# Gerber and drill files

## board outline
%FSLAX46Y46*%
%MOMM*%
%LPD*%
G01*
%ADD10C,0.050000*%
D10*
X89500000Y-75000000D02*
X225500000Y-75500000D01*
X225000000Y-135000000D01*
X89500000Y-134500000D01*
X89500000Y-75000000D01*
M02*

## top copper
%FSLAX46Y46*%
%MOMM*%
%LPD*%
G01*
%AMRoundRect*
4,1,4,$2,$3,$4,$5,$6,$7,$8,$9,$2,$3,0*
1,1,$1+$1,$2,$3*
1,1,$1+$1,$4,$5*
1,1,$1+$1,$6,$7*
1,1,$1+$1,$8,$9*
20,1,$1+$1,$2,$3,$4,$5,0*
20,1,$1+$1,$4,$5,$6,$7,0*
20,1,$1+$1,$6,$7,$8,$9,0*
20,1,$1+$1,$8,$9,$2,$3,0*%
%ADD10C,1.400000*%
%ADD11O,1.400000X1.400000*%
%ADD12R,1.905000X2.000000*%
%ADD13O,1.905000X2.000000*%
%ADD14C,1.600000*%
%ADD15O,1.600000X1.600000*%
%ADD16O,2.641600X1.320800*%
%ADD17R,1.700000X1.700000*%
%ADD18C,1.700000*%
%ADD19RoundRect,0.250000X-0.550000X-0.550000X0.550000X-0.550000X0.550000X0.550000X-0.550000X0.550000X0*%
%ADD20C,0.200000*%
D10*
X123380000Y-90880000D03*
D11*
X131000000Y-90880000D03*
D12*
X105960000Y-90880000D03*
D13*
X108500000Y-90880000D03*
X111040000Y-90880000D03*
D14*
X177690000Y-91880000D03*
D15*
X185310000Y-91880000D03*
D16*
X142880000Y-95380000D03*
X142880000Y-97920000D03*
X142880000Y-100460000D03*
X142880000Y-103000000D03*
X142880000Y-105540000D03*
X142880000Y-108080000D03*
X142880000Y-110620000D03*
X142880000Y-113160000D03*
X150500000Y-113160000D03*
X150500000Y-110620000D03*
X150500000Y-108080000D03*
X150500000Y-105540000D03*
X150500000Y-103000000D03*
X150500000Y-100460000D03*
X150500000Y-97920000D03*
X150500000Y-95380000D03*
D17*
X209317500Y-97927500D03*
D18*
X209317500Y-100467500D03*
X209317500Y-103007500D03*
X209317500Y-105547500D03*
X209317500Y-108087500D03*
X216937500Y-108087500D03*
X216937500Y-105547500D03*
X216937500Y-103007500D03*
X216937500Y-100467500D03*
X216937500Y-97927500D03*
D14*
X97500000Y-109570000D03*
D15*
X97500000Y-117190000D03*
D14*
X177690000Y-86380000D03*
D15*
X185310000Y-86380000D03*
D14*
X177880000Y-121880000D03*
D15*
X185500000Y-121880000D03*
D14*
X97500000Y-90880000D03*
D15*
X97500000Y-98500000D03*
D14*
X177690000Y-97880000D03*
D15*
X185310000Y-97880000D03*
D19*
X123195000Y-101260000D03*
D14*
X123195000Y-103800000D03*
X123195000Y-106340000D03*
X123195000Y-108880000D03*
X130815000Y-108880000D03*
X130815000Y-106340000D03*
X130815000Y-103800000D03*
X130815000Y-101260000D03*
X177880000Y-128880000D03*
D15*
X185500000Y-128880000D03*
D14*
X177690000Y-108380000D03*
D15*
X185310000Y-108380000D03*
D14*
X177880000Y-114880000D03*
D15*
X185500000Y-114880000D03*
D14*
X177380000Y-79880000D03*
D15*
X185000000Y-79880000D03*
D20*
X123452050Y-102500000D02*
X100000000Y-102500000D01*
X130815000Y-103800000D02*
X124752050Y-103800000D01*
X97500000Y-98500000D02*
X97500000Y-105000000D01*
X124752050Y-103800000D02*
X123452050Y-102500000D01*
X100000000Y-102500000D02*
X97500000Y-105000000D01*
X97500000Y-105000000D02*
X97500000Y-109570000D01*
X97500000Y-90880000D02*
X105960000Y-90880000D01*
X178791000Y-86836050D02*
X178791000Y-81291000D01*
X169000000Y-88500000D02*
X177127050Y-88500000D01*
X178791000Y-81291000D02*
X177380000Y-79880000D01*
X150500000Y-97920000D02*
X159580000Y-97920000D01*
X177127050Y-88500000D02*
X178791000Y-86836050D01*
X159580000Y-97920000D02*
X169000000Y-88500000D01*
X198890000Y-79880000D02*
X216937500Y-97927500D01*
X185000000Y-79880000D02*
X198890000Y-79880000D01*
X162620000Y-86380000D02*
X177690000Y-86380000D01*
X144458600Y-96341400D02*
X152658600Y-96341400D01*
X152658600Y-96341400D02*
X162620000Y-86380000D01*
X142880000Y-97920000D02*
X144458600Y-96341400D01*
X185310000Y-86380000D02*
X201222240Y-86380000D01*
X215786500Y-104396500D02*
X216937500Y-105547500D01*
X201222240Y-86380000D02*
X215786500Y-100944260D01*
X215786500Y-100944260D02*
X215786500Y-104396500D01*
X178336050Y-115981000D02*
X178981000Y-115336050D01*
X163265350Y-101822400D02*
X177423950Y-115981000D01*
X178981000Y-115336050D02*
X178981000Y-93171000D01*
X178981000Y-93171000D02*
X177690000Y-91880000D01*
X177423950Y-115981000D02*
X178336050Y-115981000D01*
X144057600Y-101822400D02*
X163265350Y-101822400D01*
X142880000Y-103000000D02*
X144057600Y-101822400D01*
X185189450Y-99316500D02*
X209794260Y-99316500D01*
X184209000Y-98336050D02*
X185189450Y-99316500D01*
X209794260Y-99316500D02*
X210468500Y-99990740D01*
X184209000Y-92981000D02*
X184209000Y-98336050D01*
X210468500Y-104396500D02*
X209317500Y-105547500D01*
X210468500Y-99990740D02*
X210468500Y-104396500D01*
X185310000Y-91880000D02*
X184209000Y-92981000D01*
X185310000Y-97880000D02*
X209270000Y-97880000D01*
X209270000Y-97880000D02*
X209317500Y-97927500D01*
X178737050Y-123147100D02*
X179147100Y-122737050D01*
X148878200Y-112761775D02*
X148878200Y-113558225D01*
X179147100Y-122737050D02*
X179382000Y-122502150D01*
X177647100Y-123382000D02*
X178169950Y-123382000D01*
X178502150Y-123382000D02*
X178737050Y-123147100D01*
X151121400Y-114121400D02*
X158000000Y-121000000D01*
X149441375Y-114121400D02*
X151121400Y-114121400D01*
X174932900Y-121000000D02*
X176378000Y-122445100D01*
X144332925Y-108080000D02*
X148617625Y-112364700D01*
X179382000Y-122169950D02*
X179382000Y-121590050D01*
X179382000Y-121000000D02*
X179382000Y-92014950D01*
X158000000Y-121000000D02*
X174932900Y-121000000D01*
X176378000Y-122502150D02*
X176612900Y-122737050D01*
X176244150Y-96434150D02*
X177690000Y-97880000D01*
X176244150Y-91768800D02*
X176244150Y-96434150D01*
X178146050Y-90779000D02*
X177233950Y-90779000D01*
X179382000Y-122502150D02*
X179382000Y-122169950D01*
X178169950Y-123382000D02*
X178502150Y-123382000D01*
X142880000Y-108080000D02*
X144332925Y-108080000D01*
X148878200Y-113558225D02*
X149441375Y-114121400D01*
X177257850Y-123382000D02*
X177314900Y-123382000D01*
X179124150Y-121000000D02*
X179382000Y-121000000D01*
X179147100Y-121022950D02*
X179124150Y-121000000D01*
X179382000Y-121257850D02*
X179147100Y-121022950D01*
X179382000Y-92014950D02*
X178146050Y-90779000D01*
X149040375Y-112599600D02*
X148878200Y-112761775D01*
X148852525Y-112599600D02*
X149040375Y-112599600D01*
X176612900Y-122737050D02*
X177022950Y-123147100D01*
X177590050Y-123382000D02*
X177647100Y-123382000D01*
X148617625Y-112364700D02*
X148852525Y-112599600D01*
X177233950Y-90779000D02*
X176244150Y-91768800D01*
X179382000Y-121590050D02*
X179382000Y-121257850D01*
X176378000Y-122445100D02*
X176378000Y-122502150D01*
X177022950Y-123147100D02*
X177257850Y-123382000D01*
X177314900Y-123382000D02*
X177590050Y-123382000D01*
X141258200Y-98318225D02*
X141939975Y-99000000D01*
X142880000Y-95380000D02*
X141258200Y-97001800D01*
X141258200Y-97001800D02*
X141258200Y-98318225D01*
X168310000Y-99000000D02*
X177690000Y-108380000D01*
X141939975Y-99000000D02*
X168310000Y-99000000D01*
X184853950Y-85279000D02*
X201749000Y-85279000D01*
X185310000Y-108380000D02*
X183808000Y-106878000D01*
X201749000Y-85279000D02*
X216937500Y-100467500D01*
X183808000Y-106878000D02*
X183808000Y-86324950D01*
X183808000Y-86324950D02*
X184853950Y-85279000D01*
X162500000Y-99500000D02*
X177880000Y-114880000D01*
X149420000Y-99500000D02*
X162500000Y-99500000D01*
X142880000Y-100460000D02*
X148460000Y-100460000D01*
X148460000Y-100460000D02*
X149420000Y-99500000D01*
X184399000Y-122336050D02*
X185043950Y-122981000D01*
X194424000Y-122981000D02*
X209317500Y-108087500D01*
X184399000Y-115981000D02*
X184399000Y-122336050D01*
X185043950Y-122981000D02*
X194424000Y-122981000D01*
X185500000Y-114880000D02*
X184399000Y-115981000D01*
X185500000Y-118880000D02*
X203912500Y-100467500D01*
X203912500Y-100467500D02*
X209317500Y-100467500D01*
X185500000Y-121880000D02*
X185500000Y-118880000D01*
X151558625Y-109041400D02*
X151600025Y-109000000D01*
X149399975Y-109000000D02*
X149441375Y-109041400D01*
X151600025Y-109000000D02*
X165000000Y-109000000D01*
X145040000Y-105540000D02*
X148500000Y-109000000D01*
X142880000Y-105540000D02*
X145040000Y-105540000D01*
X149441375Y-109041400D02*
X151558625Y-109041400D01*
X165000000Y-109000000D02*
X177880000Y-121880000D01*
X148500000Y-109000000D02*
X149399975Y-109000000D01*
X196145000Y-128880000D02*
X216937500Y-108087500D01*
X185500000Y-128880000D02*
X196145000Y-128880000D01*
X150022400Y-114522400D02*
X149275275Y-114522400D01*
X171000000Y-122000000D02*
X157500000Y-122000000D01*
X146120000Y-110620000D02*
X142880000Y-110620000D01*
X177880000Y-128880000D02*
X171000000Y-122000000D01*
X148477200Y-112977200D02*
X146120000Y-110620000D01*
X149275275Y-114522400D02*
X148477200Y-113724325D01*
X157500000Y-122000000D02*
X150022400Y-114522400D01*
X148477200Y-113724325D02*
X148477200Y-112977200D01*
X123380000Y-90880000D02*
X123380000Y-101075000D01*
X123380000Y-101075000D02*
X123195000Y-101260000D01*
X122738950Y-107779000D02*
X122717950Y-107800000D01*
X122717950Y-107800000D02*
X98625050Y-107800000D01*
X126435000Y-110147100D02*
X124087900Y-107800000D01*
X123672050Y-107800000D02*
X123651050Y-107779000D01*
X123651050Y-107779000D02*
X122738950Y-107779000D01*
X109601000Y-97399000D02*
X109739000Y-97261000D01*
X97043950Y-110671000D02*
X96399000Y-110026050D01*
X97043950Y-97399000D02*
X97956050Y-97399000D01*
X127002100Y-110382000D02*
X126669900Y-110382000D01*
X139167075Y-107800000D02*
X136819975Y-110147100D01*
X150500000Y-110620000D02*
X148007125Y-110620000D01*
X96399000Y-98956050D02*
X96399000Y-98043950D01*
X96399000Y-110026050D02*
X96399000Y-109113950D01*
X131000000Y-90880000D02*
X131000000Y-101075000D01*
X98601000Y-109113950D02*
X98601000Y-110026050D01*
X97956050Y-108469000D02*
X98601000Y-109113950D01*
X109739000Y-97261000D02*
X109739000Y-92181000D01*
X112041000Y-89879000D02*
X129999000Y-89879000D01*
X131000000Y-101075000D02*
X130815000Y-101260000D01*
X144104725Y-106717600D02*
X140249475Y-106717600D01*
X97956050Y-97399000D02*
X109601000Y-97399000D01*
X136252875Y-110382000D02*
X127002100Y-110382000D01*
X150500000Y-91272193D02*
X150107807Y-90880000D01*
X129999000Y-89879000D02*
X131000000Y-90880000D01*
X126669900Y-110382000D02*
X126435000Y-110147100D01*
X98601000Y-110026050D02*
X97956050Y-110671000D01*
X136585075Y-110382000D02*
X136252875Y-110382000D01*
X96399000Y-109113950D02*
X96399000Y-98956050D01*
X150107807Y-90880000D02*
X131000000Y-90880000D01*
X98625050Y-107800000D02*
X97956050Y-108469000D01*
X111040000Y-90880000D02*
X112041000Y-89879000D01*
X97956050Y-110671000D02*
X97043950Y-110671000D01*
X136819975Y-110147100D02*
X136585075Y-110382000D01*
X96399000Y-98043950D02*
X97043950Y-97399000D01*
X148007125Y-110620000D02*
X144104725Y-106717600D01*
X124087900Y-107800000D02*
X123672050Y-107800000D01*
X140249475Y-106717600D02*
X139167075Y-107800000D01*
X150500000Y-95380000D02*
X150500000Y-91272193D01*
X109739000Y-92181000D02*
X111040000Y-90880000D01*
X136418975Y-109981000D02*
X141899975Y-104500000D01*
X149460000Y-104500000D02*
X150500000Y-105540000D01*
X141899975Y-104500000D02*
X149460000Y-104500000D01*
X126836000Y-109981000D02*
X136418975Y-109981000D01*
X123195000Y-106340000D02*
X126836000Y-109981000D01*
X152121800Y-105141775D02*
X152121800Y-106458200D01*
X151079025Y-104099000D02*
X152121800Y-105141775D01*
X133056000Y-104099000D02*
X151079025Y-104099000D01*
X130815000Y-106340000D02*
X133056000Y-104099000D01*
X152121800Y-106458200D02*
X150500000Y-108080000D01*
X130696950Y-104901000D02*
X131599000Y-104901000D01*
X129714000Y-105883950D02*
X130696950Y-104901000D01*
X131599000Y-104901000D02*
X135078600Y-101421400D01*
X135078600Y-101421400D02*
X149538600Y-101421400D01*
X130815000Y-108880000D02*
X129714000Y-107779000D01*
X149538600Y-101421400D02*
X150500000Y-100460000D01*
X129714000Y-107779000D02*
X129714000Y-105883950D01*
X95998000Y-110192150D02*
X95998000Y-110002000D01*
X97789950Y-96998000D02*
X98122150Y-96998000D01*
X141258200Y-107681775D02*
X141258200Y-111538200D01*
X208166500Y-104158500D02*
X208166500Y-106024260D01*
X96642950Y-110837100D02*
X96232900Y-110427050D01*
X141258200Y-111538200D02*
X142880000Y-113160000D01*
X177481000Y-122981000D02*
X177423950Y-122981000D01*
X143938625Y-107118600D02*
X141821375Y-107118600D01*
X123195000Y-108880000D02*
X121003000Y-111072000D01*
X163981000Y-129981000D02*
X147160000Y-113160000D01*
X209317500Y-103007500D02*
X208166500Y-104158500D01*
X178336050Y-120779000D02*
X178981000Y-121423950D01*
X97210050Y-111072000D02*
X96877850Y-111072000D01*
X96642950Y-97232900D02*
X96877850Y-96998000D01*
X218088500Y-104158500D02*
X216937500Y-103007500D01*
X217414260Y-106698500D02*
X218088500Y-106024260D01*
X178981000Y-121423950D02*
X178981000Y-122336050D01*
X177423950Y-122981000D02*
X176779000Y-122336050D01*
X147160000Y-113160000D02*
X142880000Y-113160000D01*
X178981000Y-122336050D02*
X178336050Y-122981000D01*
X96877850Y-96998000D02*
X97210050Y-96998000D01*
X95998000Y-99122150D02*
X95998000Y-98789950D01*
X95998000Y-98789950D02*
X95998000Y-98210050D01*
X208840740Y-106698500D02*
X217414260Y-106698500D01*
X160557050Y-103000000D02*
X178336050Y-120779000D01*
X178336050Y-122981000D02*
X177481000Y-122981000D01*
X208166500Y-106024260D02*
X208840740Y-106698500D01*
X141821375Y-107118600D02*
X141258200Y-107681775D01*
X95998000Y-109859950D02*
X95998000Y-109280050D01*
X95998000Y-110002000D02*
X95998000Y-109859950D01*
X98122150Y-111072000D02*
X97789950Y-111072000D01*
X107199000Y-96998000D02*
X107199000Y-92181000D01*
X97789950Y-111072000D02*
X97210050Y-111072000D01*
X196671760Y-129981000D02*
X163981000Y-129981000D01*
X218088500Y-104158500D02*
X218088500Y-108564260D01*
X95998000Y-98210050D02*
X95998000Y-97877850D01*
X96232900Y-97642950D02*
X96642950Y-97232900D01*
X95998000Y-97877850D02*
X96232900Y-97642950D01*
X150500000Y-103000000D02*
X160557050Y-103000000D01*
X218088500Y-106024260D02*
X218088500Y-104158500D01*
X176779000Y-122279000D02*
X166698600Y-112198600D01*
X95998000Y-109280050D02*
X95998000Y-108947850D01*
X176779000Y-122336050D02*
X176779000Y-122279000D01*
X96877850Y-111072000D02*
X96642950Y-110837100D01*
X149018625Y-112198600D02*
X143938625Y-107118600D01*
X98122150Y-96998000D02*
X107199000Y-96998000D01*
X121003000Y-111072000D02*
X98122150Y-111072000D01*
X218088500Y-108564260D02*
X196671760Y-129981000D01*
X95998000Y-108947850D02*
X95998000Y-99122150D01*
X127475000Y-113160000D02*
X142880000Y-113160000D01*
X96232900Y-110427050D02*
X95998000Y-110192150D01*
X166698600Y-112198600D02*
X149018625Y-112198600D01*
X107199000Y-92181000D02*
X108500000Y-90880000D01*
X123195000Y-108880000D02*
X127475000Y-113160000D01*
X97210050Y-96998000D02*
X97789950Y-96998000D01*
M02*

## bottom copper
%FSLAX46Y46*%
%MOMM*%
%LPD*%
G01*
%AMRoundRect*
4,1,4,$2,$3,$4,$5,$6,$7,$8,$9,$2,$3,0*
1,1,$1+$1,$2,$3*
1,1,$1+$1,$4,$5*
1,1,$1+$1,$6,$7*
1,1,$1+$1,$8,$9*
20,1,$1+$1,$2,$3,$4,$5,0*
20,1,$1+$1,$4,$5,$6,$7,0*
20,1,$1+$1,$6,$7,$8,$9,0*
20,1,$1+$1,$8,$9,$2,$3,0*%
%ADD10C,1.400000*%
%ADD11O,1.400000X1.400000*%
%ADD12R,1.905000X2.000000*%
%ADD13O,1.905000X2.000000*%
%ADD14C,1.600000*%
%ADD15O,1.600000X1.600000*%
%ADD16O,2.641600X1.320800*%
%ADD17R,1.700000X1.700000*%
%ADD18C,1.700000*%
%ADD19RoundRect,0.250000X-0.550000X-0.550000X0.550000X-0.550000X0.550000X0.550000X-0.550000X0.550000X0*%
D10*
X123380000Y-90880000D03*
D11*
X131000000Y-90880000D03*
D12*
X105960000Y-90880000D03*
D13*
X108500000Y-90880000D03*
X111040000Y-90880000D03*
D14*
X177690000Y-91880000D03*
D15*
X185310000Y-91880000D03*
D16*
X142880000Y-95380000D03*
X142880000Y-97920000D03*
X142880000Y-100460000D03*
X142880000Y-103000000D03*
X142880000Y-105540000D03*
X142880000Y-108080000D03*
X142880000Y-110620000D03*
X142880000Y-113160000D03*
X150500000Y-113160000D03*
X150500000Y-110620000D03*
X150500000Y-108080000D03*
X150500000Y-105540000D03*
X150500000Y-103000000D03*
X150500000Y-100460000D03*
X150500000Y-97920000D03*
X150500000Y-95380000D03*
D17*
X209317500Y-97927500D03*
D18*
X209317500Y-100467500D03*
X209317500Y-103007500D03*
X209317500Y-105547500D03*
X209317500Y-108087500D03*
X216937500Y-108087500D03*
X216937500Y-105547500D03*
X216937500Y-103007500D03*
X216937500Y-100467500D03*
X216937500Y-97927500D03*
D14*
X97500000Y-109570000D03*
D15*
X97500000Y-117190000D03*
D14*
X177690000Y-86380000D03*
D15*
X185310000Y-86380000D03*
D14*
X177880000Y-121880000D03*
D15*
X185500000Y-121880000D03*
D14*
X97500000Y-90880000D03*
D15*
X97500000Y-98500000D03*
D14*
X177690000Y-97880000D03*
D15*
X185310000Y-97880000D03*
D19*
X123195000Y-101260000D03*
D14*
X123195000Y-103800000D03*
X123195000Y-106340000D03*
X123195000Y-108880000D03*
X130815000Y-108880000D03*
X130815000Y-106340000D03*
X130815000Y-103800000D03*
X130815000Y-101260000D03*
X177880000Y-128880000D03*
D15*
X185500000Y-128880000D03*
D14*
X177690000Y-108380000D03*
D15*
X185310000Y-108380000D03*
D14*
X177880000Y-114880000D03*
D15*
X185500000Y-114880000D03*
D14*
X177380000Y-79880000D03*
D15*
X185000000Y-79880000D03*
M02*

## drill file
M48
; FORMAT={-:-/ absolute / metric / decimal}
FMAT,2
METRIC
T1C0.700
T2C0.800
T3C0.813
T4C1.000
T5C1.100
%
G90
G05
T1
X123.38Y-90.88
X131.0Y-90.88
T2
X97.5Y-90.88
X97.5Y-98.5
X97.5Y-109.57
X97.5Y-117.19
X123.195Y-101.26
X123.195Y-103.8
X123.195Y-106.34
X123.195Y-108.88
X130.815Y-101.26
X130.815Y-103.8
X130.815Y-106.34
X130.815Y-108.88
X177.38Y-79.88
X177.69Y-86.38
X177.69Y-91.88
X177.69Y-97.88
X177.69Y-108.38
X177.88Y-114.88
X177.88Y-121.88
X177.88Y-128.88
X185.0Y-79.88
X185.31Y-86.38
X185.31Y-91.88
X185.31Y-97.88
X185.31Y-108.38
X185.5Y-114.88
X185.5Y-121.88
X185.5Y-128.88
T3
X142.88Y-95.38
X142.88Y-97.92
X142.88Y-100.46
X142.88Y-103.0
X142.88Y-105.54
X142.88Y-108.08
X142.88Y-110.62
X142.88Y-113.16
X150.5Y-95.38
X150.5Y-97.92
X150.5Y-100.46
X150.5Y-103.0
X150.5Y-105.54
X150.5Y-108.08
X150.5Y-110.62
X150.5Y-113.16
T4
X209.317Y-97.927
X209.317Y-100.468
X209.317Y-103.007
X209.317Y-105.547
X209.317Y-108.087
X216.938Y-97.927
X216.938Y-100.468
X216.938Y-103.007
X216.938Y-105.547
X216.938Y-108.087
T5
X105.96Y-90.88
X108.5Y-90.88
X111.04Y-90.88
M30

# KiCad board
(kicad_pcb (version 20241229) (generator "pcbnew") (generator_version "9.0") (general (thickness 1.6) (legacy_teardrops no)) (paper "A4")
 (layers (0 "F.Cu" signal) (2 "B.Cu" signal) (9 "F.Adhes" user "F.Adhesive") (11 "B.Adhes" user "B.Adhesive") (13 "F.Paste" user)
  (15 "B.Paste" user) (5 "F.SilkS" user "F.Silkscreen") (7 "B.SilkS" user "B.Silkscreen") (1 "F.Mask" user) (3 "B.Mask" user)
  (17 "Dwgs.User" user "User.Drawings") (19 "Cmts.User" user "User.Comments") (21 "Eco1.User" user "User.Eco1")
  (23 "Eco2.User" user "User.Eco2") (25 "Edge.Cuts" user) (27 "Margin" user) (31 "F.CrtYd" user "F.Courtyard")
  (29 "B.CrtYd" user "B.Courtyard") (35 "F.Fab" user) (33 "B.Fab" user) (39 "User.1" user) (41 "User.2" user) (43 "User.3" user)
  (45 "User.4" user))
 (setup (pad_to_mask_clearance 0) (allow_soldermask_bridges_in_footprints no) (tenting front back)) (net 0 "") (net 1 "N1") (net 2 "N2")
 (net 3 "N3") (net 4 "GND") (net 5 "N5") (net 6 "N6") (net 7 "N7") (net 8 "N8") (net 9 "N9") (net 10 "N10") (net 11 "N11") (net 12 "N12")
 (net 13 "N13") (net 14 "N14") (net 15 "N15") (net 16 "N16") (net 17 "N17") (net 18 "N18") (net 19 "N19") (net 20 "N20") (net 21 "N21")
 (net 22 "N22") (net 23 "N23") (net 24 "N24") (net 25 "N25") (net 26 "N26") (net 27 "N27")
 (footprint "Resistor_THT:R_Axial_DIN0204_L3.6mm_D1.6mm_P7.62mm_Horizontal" (layer "F.Cu") (at 123.38 90.88)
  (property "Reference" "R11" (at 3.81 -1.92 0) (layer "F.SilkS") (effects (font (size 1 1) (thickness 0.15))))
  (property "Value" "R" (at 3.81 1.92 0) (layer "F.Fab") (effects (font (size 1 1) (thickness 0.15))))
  (pad "1" thru_hole circle (at 0 0) (size 1.4 1.4) (drill 0.7) (layers "*.Cu" "*.Mask") (remove_unused_layers no) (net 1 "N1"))
  (pad "2" thru_hole oval (at 7.62 0) (size 1.4 1.4) (drill 0.7) (layers "*.Cu" "*.Mask") (remove_unused_layers no) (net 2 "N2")))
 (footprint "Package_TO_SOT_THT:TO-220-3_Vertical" (layer "F.Cu") (at 105.96 90.88)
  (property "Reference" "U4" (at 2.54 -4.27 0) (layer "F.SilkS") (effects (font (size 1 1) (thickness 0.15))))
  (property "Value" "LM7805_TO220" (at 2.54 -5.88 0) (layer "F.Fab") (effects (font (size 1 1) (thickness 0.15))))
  (pad "1" thru_hole rect (at 0 0) (size 1.905 2) (drill 1.1) (layers "*.Cu" "*.Mask") (remove_unused_layers no) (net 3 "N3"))
  (pad "2" thru_hole oval (at 2.54 0) (size 1.905 2) (drill 1.1) (layers "*.Cu" "*.Mask") (remove_unused_layers no) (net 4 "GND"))
  (pad "3" thru_hole oval (at 5.08 0) (size 1.905 2) (drill 1.1) (layers "*.Cu" "*.Mask") (remove_unused_layers no) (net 2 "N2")))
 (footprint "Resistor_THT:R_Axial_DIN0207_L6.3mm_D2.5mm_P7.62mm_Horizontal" (layer "F.Cu") (at 177.69 91.88)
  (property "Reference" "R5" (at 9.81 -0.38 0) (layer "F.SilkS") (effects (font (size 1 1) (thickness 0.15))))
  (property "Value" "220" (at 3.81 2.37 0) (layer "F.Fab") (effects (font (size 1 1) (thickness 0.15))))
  (pad "1" thru_hole circle (at 0 0) (size 1.6 1.6) (drill 0.8) (layers "*.Cu" "*.Mask") (remove_unused_layers no) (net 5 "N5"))
  (pad "2" thru_hole oval (at 7.62 0) (size 1.6 1.6) (drill 0.8) (layers "*.Cu" "*.Mask") (remove_unused_layers no) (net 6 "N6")))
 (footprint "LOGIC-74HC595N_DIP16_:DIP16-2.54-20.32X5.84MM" (layer "F.Cu") (at 146.69 104.27 -90)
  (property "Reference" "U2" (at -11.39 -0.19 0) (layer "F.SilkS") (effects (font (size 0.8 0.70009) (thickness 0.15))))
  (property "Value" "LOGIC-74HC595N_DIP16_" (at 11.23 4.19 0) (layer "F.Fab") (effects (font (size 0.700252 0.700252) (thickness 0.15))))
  (pad "1" thru_hole oval (at -8.89 3.81 270) (size 1.3208 2.6416) (drill 0.8128) (layers "*.Cu" "*.Mask") (remove_unused_layers no)
   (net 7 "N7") (solder_mask_margin 0.102))
  (pad "2" thru_hole oval (at -6.35 3.81 270) (size 1.3208 2.6416) (drill 0.8128) (layers "*.Cu" "*.Mask") (remove_unused_layers no)
   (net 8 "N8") (solder_mask_margin 0.102))
  (pad "3" thru_hole oval (at -3.81 3.81 270) (size 1.3208 2.6416) (drill 0.8128) (layers "*.Cu" "*.Mask") (remove_unused_layers no)
   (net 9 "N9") (solder_mask_margin 0.102))
  (pad "4" thru_hole oval (at -1.27 3.81 270) (size 1.3208 2.6416) (drill 0.8128) (layers "*.Cu" "*.Mask") (remove_unused_layers no)
   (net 5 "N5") (solder_mask_margin 0.102))
  (pad "5" thru_hole oval (at 1.27 3.81 270) (size 1.3208 2.6416) (drill 0.8128) (layers "*.Cu" "*.Mask") (remove_unused_layers no)
   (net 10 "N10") (solder_mask_margin 0.102))
  (pad "6" thru_hole oval (at 3.81 3.81 270) (size 1.3208 2.6416) (drill 0.8128) (layers "*.Cu" "*.Mask") (remove_unused_layers no)
   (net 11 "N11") (solder_mask_margin 0.102))
  (pad "7" thru_hole oval (at 6.35 3.81 270) (size 1.3208 2.6416) (drill 0.8128) (layers "*.Cu" "*.Mask") (remove_unused_layers no)
   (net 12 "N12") (solder_mask_margin 0.102))
  (pad "8" thru_hole oval (at 8.89 3.81 270) (size 1.3208 2.6416) (drill 0.8128) (layers "*.Cu" "*.Mask") (remove_unused_layers no)
   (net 4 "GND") (solder_mask_margin 0.102))
  (pad "9" thru_hole oval (at 8.89 -3.81 270) (size 1.3208 2.6416) (drill 0.8128) (layers "*.Cu" "*.Mask") (remove_unused_layers no)
   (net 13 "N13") (solder_mask_margin 0.102))
  (pad "10" thru_hole oval (at 6.35 -3.81 270) (size 1.3208 2.6416) (drill 0.8128) (layers "*.Cu" "*.Mask") (remove_unused_layers no)
   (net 2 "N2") (solder_mask_margin 0.102))
  (pad "11" thru_hole oval (at 3.81 -3.81 270) (size 1.3208 2.6416) (drill 0.8128) (layers "*.Cu" "*.Mask") (remove_unused_layers no)
   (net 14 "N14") (solder_mask_margin 0.102))
  (pad "12" thru_hole oval (at 1.27 -3.81 270) (size 1.3208 2.6416) (drill 0.8128) (layers "*.Cu" "*.Mask") (remove_unused_layers no)
   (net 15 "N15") (solder_mask_margin 0.102))
  (pad "13" thru_hole oval (at -1.27 -3.81 270) (size 1.3208 2.6416) (drill 0.8128) (layers "*.Cu" "*.Mask") (remove_unused_layers no)
   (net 4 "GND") (solder_mask_margin 0.102))
  (pad "14" thru_hole oval (at -3.81 -3.81 270) (size 1.3208 2.6416) (drill 0.8128) (layers "*.Cu" "*.Mask") (remove_unused_layers no)
   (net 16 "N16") (solder_mask_margin 0.102))
  (pad "15" thru_hole oval (at -6.35 -3.81 270) (size 1.3208 2.6416) (drill 0.8128) (layers "*.Cu" "*.Mask") (remove_unused_layers no)
   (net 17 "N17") (solder_mask_margin 0.102))
  (pad "16" thru_hole oval (at -8.89 -3.81 270) (size 1.3208 2.6416) (drill 0.8128) (layers "*.Cu" "*.Mask") (remove_unused_layers no)
   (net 2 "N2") (solder_mask_margin 0.102)))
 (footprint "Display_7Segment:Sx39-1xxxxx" (layer "F.Cu") (at 209.3175 97.9275)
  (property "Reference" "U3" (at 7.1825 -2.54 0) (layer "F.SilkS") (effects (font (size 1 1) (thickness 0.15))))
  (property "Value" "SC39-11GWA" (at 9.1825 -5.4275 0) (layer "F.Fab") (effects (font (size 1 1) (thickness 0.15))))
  (pad "1" thru_hole rect (at 0 0) (size 1.7 1.7) (drill 1) (layers "*.Cu" "*.Mask") (remove_unused_layers no) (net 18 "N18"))
  (pad "2" thru_hole circle (at 0 2.54) (size 1.7 1.7) (drill 1) (layers "*.Cu" "*.Mask") (remove_unused_layers no) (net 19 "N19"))
  (pad "3" thru_hole circle (at 0 5.08) (size 1.7 1.7) (drill 1) (layers "*.Cu" "*.Mask") (remove_unused_layers no) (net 4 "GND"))
  (pad "4" thru_hole circle (at 0 7.62) (size 1.7 1.7) (drill 1) (layers "*.Cu" "*.Mask") (remove_unused_layers no) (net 6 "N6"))
  (pad "5" thru_hole circle (at 0 10.16) (size 1.7 1.7) (drill 1) (layers "*.Cu" "*.Mask") (remove_unused_layers no) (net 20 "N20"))
  (pad "6" thru_hole circle (at 7.62 10.16) (size 1.7 1.7) (drill 1) (layers "*.Cu" "*.Mask") (remove_unused_layers no) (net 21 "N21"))
  (pad "7" thru_hole circle (at 7.62 7.62) (size 1.7 1.7) (drill 1) (layers "*.Cu" "*.Mask") (remove_unused_layers no) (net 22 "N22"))
  (pad "8" thru_hole circle (at 7.62 5.08) (size 1.7 1.7) (drill 1) (layers "*.Cu" "*.Mask") (remove_unused_layers no) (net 4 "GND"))
  (pad "9" thru_hole circle (at 7.62 2.54) (size 1.7 1.7) (drill 1) (layers "*.Cu" "*.Mask") (remove_unused_layers no) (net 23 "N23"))
  (pad "10" thru_hole circle (at 7.62 0) (size 1.7 1.7) (drill 1) (layers "*.Cu" "*.Mask") (remove_unused_layers no) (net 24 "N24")))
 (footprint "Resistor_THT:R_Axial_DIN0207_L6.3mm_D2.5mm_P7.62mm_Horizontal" (layer "F.Cu") (at 97.5 109.57 -90)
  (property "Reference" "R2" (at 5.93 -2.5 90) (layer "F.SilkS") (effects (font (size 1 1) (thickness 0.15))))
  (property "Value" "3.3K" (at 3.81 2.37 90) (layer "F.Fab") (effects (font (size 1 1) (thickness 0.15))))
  (pad "1" thru_hole circle (at 0 0 270) (size 1.6 1.6) (drill 0.8) (layers "*.Cu" "*.Mask") (remove_unused_layers no) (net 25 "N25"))
  (pad "2" thru_hole oval (at 7.62 0 270) (size 1.6 1.6) (drill 0.8) (layers "*.Cu" "*.Mask") (remove_unused_layers no) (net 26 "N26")))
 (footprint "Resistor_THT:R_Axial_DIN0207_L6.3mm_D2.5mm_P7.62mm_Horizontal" (layer "F.Cu") (at 177.69 86.38)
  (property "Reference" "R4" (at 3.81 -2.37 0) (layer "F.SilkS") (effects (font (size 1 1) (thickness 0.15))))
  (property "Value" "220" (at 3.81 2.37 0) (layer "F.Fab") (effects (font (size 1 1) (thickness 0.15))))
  (pad "1" thru_hole circle (at 0 0) (size 1.6 1.6) (drill 0.8) (layers "*.Cu" "*.Mask") (remove_unused_layers no) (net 8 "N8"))
  (pad "2" thru_hole oval (at 7.62 0) (size 1.6 1.6) (drill 0.8) (layers "*.Cu" "*.Mask") (remove_unused_layers no) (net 22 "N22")))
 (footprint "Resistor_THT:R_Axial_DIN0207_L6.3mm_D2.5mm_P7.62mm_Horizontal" (layer "F.Cu") (at 177.88 121.88)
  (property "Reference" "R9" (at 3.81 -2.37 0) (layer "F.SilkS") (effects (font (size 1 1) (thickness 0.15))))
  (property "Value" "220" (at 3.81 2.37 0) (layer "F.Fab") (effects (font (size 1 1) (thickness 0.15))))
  (pad "1" thru_hole circle (at 0 0) (size 1.6 1.6) (drill 0.8) (layers "*.Cu" "*.Mask") (remove_unused_layers no) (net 10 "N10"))
  (pad "2" thru_hole oval (at 7.62 0) (size 1.6 1.6) (drill 0.8) (layers "*.Cu" "*.Mask") (remove_unused_layers no) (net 19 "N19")))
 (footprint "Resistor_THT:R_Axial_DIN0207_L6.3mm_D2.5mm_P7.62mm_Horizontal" (layer "F.Cu") (at 97.5 90.88 -90)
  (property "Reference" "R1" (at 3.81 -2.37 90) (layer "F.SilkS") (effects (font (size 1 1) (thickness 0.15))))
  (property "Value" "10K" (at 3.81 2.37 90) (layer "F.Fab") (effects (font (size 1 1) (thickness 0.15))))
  (pad "1" thru_hole circle (at 0 0 270) (size 1.6 1.6) (drill 0.8) (layers "*.Cu" "*.Mask") (remove_unused_layers no) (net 3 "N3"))
  (pad "2" thru_hole oval (at 7.62 0 270) (size 1.6 1.6) (drill 0.8) (layers "*.Cu" "*.Mask") (remove_unused_layers no) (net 25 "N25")))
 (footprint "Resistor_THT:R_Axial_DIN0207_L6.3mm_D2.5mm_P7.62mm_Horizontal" (layer "F.Cu") (at 177.69 97.88)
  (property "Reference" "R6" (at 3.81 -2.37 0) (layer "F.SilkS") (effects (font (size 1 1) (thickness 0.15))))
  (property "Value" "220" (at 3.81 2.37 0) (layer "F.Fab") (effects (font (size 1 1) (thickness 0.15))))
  (pad "1" thru_hole circle (at 0 0) (size 1.6 1.6) (drill 0.8) (layers "*.Cu" "*.Mask") (remove_unused_layers no) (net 11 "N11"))
  (pad "2" thru_hole oval (at 7.62 0) (size 1.6 1.6) (drill 0.8) (layers "*.Cu" "*.Mask") (remove_unused_layers no) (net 18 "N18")))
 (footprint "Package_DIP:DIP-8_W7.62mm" (layer "F.Cu") (at 123.195 101.26)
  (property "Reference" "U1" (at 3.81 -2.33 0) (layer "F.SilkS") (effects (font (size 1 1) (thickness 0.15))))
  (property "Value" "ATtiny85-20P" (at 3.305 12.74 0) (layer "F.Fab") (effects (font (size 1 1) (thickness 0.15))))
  (pad "1" thru_hole roundrect (at 0 0) (size 1.6 1.6) (drill 0.8) (layers "*.Cu" "*.Mask") (remove_unused_layers no)
   (roundrect_rratio 0.15625) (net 1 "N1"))
  (pad "2" thru_hole circle (at 0 2.54) (size 1.6 1.6) (drill 0.8) (layers "*.Cu" "*.Mask") (remove_unused_layers no) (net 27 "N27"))
  (pad "3" thru_hole circle (at 0 5.08) (size 1.6 1.6) (drill 0.8) (layers "*.Cu" "*.Mask") (remove_unused_layers no) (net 15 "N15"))
  (pad "4" thru_hole circle (at 0 7.62) (size 1.6 1.6) (drill 0.8) (layers "*.Cu" "*.Mask") (remove_unused_layers no) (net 4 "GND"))
  (pad "5" thru_hole circle (at 7.62 7.62) (size 1.6 1.6) (drill 0.8) (layers "*.Cu" "*.Mask") (remove_unused_layers no) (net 16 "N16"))
  (pad "6" thru_hole circle (at 7.62 5.08) (size 1.6 1.6) (drill 0.8) (layers "*.Cu" "*.Mask") (remove_unused_layers no) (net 14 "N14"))
  (pad "7" thru_hole circle (at 7.62 2.54) (size 1.6 1.6) (drill 0.8) (layers "*.Cu" "*.Mask") (remove_unused_layers no) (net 25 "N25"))
  (pad "8" thru_hole circle (at 7.62 0) (size 1.6 1.6) (drill 0.8) (layers "*.Cu" "*.Mask") (remove_unused_layers no) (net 2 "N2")))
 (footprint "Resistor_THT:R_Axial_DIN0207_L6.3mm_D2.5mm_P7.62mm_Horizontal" (layer "F.Cu") (at 177.88 128.88)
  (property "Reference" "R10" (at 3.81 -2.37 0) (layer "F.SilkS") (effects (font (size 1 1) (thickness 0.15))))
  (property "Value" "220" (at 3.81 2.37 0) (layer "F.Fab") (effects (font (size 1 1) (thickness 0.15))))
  (pad "1" thru_hole circle (at 0 0) (size 1.6 1.6) (drill 0.8) (layers "*.Cu" "*.Mask") (remove_unused_layers no) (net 12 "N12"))
  (pad "2" thru_hole oval (at 7.62 0) (size 1.6 1.6) (drill 0.8) (layers "*.Cu" "*.Mask") (remove_unused_layers no) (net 21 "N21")))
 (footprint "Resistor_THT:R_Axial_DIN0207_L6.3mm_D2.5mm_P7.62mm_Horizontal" (layer "F.Cu") (at 177.69 108.38)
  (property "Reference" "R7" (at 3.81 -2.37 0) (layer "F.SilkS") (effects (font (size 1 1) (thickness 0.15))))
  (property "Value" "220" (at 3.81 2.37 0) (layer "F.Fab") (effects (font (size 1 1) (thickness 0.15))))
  (pad "1" thru_hole circle (at 0 0) (size 1.6 1.6) (drill 0.8) (layers "*.Cu" "*.Mask") (remove_unused_layers no) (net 7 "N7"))
  (pad "2" thru_hole oval (at 7.62 0) (size 1.6 1.6) (drill 0.8) (layers "*.Cu" "*.Mask") (remove_unused_layers no) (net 23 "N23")))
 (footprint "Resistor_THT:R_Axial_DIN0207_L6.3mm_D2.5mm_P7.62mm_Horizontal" (layer "F.Cu") (at 177.88 114.88)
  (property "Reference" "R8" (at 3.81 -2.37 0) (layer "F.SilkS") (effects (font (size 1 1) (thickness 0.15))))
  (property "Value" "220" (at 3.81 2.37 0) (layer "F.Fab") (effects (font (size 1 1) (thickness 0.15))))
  (pad "1" thru_hole circle (at 0 0) (size 1.6 1.6) (drill 0.8) (layers "*.Cu" "*.Mask") (remove_unused_layers no) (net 9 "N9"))
  (pad "2" thru_hole oval (at 7.62 0) (size 1.6 1.6) (drill 0.8) (layers "*.Cu" "*.Mask") (remove_unused_layers no) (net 20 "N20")))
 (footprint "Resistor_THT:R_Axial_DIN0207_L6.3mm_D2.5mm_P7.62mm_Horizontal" (layer "F.Cu") (at 177.38 79.88)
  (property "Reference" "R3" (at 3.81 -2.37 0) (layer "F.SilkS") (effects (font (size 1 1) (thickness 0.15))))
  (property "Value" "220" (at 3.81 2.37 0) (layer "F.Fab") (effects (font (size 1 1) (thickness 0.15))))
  (pad "1" thru_hole circle (at 0 0) (size 1.6 1.6) (drill 0.8) (layers "*.Cu" "*.Mask") (remove_unused_layers no) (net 17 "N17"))
  (pad "2" thru_hole oval (at 7.62 0) (size 1.6 1.6) (drill 0.8) (layers "*.Cu" "*.Mask") (remove_unused_layers no) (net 24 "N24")))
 (gr_poly (pts (xy 89.5 75) (xy 225.5 75.5) (xy 225 135) (xy 89.5 134.5)) (stroke (width 0.05) (type solid)) (fill no) (layer "Edge.Cuts"))
 (segment (start 123.45205 102.5) (end 100 102.5) (width 0.2) (layer "F.Cu") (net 25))
 (segment (start 130.815 103.8) (end 124.75205 103.8) (width 0.2) (layer "F.Cu") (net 25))
 (segment (start 97.5 98.5) (end 97.5 105) (width 0.2) (layer "F.Cu") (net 25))
 (segment (start 124.75205 103.8) (end 123.45205 102.5) (width 0.2) (layer "F.Cu") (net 25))
 (segment (start 100 102.5) (end 97.5 105) (width 0.2) (layer "F.Cu") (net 25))
 (segment (start 97.5 105) (end 97.5 109.57) (width 0.2) (layer "F.Cu") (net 25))
 (segment (start 97.5 90.88) (end 105.96 90.88) (width 0.2) (layer "F.Cu") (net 3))
 (segment (start 178.791 86.83605) (end 178.791 81.291) (width 0.2) (layer "F.Cu") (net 17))
 (segment (start 169 88.5) (end 177.12705 88.5) (width 0.2) (layer "F.Cu") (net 17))
 (segment (start 178.791 81.291) (end 177.38 79.88) (width 0.2) (layer "F.Cu") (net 17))
 (segment (start 150.5 97.92) (end 159.58 97.92) (width 0.2) (layer "F.Cu") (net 17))
 (segment (start 177.12705 88.5) (end 178.791 86.83605) (width 0.2) (layer "F.Cu") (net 17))
 (segment (start 159.58 97.92) (end 169 88.5) (width 0.2) (layer "F.Cu") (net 17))
 (segment (start 198.89 79.88) (end 216.9375 97.9275) (width 0.2) (layer "F.Cu") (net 24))
 (segment (start 185 79.88) (end 198.89 79.88) (width 0.2) (layer "F.Cu") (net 24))
 (segment (start 162.62 86.38) (end 177.69 86.38) (width 0.2) (layer "F.Cu") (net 8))
 (segment (start 144.4586 96.3414) (end 152.6586 96.3414) (width 0.2) (layer "F.Cu") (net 8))
 (segment (start 152.6586 96.3414) (end 162.62 86.38) (width 0.2) (layer "F.Cu") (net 8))
 (segment (start 142.88 97.92) (end 144.4586 96.3414) (width 0.2) (layer "F.Cu") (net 8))
 (segment (start 185.31 86.38) (end 201.22224 86.38) (width 0.2) (layer "F.Cu") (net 22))
 (segment (start 215.7865 104.3965) (end 216.9375 105.5475) (width 0.2) (layer "F.Cu") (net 22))
 (segment (start 201.22224 86.38) (end 215.7865 100.94426) (width 0.2) (layer "F.Cu") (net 22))
 (segment (start 215.7865 100.94426) (end 215.7865 104.3965) (width 0.2) (layer "F.Cu") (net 22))
 (segment (start 178.33605 115.981) (end 178.981 115.33605) (width 0.2) (layer "F.Cu") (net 5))
 (segment (start 163.26535 101.8224) (end 177.42395 115.981) (width 0.2) (layer "F.Cu") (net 5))
 (segment (start 178.981 115.33605) (end 178.981 93.171) (width 0.2) (layer "F.Cu") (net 5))
 (segment (start 178.981 93.171) (end 177.69 91.88) (width 0.2) (layer "F.Cu") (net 5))
 (segment (start 177.42395 115.981) (end 178.33605 115.981) (width 0.2) (layer "F.Cu") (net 5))
 (segment (start 144.0576 101.8224) (end 163.26535 101.8224) (width 0.2) (layer "F.Cu") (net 5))
 (segment (start 142.88 103) (end 144.0576 101.8224) (width 0.2) (layer "F.Cu") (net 5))
 (segment (start 185.18945 99.3165) (end 209.79426 99.3165) (width 0.2) (layer "F.Cu") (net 6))
 (segment (start 184.209 98.33605) (end 185.18945 99.3165) (width 0.2) (layer "F.Cu") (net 6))
 (segment (start 209.79426 99.3165) (end 210.4685 99.99074) (width 0.2) (layer "F.Cu") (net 6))
 (segment (start 184.209 92.981) (end 184.209 98.33605) (width 0.2) (layer "F.Cu") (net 6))
 (segment (start 210.4685 104.3965) (end 209.3175 105.5475) (width 0.2) (layer "F.Cu") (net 6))
 (segment (start 210.4685 99.99074) (end 210.4685 104.3965) (width 0.2) (layer "F.Cu") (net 6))
 (segment (start 185.31 91.88) (end 184.209 92.981) (width 0.2) (layer "F.Cu") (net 6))
 (segment (start 185.31 97.88) (end 209.27 97.88) (width 0.2) (layer "F.Cu") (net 18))
 (segment (start 209.27 97.88) (end 209.3175 97.9275) (width 0.2) (layer "F.Cu") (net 18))
 (segment (start 178.73705 123.1471) (end 179.1471 122.73705) (width 0.2) (layer "F.Cu") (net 11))
 (segment (start 148.8782 112.761775) (end 148.8782 113.558225) (width 0.2) (layer "F.Cu") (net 11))
 (segment (start 179.1471 122.73705) (end 179.382 122.50215) (width 0.2) (layer "F.Cu") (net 11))
 (segment (start 177.6471 123.382) (end 178.16995 123.382) (width 0.2) (layer "F.Cu") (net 11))
 (segment (start 178.50215 123.382) (end 178.73705 123.1471) (width 0.2) (layer "F.Cu") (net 11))
 (segment (start 151.1214 114.1214) (end 158 121) (width 0.2) (layer "F.Cu") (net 11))
 (segment (start 149.441375 114.1214) (end 151.1214 114.1214) (width 0.2) (layer "F.Cu") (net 11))
 (segment (start 174.9329 121) (end 176.378 122.4451) (width 0.2) (layer "F.Cu") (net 11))
 (segment (start 144.332925 108.08) (end 148.617625 112.3647) (width 0.2) (layer "F.Cu") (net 11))
 (segment (start 179.382 122.16995) (end 179.382 121.59005) (width 0.2) (layer "F.Cu") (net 11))
 (segment (start 179.382 121) (end 179.382 92.01495) (width 0.2) (layer "F.Cu") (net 11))
 (segment (start 158 121) (end 174.9329 121) (width 0.2) (layer "F.Cu") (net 11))
 (segment (start 176.378 122.50215) (end 176.6129 122.73705) (width 0.2) (layer "F.Cu") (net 11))
 (segment (start 176.24415 96.43415) (end 177.69 97.88) (width 0.2) (layer "F.Cu") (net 11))
 (segment (start 176.24415 91.7688) (end 176.24415 96.43415) (width 0.2) (layer "F.Cu") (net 11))
 (segment (start 178.14605 90.779) (end 177.23395 90.779) (width 0.2) (layer "F.Cu") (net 11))
 (segment (start 179.382 122.50215) (end 179.382 122.16995) (width 0.2) (layer "F.Cu") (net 11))
 (segment (start 178.16995 123.382) (end 178.50215 123.382) (width 0.2) (layer "F.Cu") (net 11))
 (segment (start 142.88 108.08) (end 144.332925 108.08) (width 0.2) (layer "F.Cu") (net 11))
 (segment (start 148.8782 113.558225) (end 149.441375 114.1214) (width 0.2) (layer "F.Cu") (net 11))
 (segment (start 177.25785 123.382) (end 177.3149 123.382) (width 0.2) (layer "F.Cu") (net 11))
 (segment (start 179.12415 121) (end 179.382 121) (width 0.2) (layer "F.Cu") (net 11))
 (segment (start 179.1471 121.02295) (end 179.12415 121) (width 0.2) (layer "F.Cu") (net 11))
 (segment (start 179.382 121.25785) (end 179.1471 121.02295) (width 0.2) (layer "F.Cu") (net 11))
 (segment (start 179.382 92.01495) (end 178.14605 90.779) (width 0.2) (layer "F.Cu") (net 11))
 (segment (start 149.040375 112.5996) (end 148.8782 112.761775) (width 0.2) (layer "F.Cu") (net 11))
 (segment (start 148.852525 112.5996) (end 149.040375 112.5996) (width 0.2) (layer "F.Cu") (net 11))
 (segment (start 176.6129 122.73705) (end 177.02295 123.1471) (width 0.2) (layer "F.Cu") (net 11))
 (segment (start 177.59005 123.382) (end 177.6471 123.382) (width 0.2) (layer "F.Cu") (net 11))
 (segment (start 148.617625 112.3647) (end 148.852525 112.5996) (width 0.2) (layer "F.Cu") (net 11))
 (segment (start 177.23395 90.779) (end 176.24415 91.7688) (width 0.2) (layer "F.Cu") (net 11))
 (segment (start 179.382 121.59005) (end 179.382 121.25785) (width 0.2) (layer "F.Cu") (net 11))
 (segment (start 176.378 122.4451) (end 176.378 122.50215) (width 0.2) (layer "F.Cu") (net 11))
 (segment (start 177.02295 123.1471) (end 177.25785 123.382) (width 0.2) (layer "F.Cu") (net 11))
 (segment (start 177.3149 123.382) (end 177.59005 123.382) (width 0.2) (layer "F.Cu") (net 11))
 (segment (start 141.2582 98.318225) (end 141.939975 99) (width 0.2) (layer "F.Cu") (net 7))
 (segment (start 142.88 95.38) (end 141.2582 97.0018) (width 0.2) (layer "F.Cu") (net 7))
 (segment (start 141.2582 97.0018) (end 141.2582 98.318225) (width 0.2) (layer "F.Cu") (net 7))
 (segment (start 168.31 99) (end 177.69 108.38) (width 0.2) (layer "F.Cu") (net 7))
 (segment (start 141.939975 99) (end 168.31 99) (width 0.2) (layer "F.Cu") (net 7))
 (segment (start 184.85395 85.279) (end 201.749 85.279) (width 0.2) (layer "F.Cu") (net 23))
 (segment (start 185.31 108.38) (end 183.808 106.878) (width 0.2) (layer "F.Cu") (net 23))
 (segment (start 201.749 85.279) (end 216.9375 100.4675) (width 0.2) (layer "F.Cu") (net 23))
 (segment (start 183.808 106.878) (end 183.808 86.32495) (width 0.2) (layer "F.Cu") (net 23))
 (segment (start 183.808 86.32495) (end 184.85395 85.279) (width 0.2) (layer "F.Cu") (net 23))
 (segment (start 162.5 99.5) (end 177.88 114.88) (width 0.2) (layer "F.Cu") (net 9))
 (segment (start 149.42 99.5) (end 162.5 99.5) (width 0.2) (layer "F.Cu") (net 9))
 (segment (start 142.88 100.46) (end 148.46 100.46) (width 0.2) (layer "F.Cu") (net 9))
 (segment (start 148.46 100.46) (end 149.42 99.5) (width 0.2) (layer "F.Cu") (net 9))
 (segment (start 184.399 122.33605) (end 185.04395 122.981) (width 0.2) (layer "F.Cu") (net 20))
 (segment (start 194.424 122.981) (end 209.3175 108.0875) (width 0.2) (layer "F.Cu") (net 20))
 (segment (start 184.399 115.981) (end 184.399 122.33605) (width 0.2) (layer "F.Cu") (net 20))
 (segment (start 185.04395 122.981) (end 194.424 122.981) (width 0.2) (layer "F.Cu") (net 20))
 (segment (start 185.5 114.88) (end 184.399 115.981) (width 0.2) (layer "F.Cu") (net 20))
 (segment (start 185.5 118.88) (end 203.9125 100.4675) (width 0.2) (layer "F.Cu") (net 19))
 (segment (start 203.9125 100.4675) (end 209.3175 100.4675) (width 0.2) (layer "F.Cu") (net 19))
 (segment (start 185.5 121.88) (end 185.5 118.88) (width 0.2) (layer "F.Cu") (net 19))
 (segment (start 151.558625 109.0414) (end 151.600025 109) (width 0.2) (layer "F.Cu") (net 10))
 (segment (start 149.399975 109) (end 149.441375 109.0414) (width 0.2) (layer "F.Cu") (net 10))
 (segment (start 151.600025 109) (end 165 109) (width 0.2) (layer "F.Cu") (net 10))
 (segment (start 145.04 105.54) (end 148.5 109) (width 0.2) (layer "F.Cu") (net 10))
 (segment (start 142.88 105.54) (end 145.04 105.54) (width 0.2) (layer "F.Cu") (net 10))
 (segment (start 149.441375 109.0414) (end 151.558625 109.0414) (width 0.2) (layer "F.Cu") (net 10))
 (segment (start 165 109) (end 177.88 121.88) (width 0.2) (layer "F.Cu") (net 10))
 (segment (start 148.5 109) (end 149.399975 109) (width 0.2) (layer "F.Cu") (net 10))
 (segment (start 196.145 128.88) (end 216.9375 108.0875) (width 0.2) (layer "F.Cu") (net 21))
 (segment (start 185.5 128.88) (end 196.145 128.88) (width 0.2) (layer "F.Cu") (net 21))
 (segment (start 150.0224 114.5224) (end 149.275275 114.5224) (width 0.2) (layer "F.Cu") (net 12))
 (segment (start 171 122) (end 157.5 122) (width 0.2) (layer "F.Cu") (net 12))
 (segment (start 146.12 110.62) (end 142.88 110.62) (width 0.2) (layer "F.Cu") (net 12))
 (segment (start 177.88 128.88) (end 171 122) (width 0.2) (layer "F.Cu") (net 12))
 (segment (start 148.4772 112.9772) (end 146.12 110.62) (width 0.2) (layer "F.Cu") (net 12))
 (segment (start 149.275275 114.5224) (end 148.4772 113.724325) (width 0.2) (layer "F.Cu") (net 12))
 (segment (start 157.5 122) (end 150.0224 114.5224) (width 0.2) (layer "F.Cu") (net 12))
 (segment (start 148.4772 113.724325) (end 148.4772 112.9772) (width 0.2) (layer "F.Cu") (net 12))
 (segment (start 123.38 90.88) (end 123.38 101.075) (width 0.2) (layer "F.Cu") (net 1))
 (segment (start 123.38 101.075) (end 123.195 101.26) (width 0.2) (layer "F.Cu") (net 1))
 (segment (start 122.73895 107.779) (end 122.71795 107.8) (width 0.2) (layer "F.Cu") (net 2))
 (segment (start 122.71795 107.8) (end 98.62505 107.8) (width 0.2) (layer "F.Cu") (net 2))
 (segment (start 126.435 110.1471) (end 124.0879 107.8) (width 0.2) (layer "F.Cu") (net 2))
 (segment (start 123.67205 107.8) (end 123.65105 107.779) (width 0.2) (layer "F.Cu") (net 2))
 (segment (start 123.65105 107.779) (end 122.73895 107.779) (width 0.2) (layer "F.Cu") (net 2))
 (segment (start 109.601 97.399) (end 109.739 97.261) (width 0.2) (layer "F.Cu") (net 2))
 (segment (start 97.04395 110.671) (end 96.399 110.02605) (width 0.2) (layer "F.Cu") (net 2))
 (segment (start 97.04395 97.399) (end 97.95605 97.399) (width 0.2) (layer "F.Cu") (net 2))
 (segment (start 127.0021 110.382) (end 126.6699 110.382) (width 0.2) (layer "F.Cu") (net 2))
 (segment (start 139.167075 107.8) (end 136.819975 110.1471) (width 0.2) (layer "F.Cu") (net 2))
 (segment (start 150.5 110.62) (end 148.007125 110.62) (width 0.2) (layer "F.Cu") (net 2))
 (segment (start 96.399 98.95605) (end 96.399 98.04395) (width 0.2) (layer "F.Cu") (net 2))
 (segment (start 96.399 110.02605) (end 96.399 109.11395) (width 0.2) (layer "F.Cu") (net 2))
 (segment (start 131 90.88) (end 131 101.075) (width 0.2) (layer "F.Cu") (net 2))
 (segment (start 98.601 109.11395) (end 98.601 110.02605) (width 0.2) (layer "F.Cu") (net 2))
 (segment (start 97.95605 108.469) (end 98.601 109.11395) (width 0.2) (layer "F.Cu") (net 2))
 (segment (start 109.739 97.261) (end 109.739 92.181) (width 0.2) (layer "F.Cu") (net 2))
 (segment (start 112.041 89.879) (end 129.999 89.879) (width 0.2) (layer "F.Cu") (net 2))
 (segment (start 131 101.075) (end 130.815 101.26) (width 0.2) (layer "F.Cu") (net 2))
 (segment (start 144.104725 106.7176) (end 140.249475 106.7176) (width 0.2) (layer "F.Cu") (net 2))
 (segment (start 97.95605 97.399) (end 109.601 97.399) (width 0.2) (layer "F.Cu") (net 2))
 (segment (start 136.252875 110.382) (end 127.0021 110.382) (width 0.2) (layer "F.Cu") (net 2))
 (segment (start 150.5 91.272193) (end 150.107807 90.88) (width 0.2) (layer "F.Cu") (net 2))
 (segment (start 129.999 89.879) (end 131 90.88) (width 0.2) (layer "F.Cu") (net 2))
 (segment (start 126.6699 110.382) (end 126.435 110.1471) (width 0.2) (layer "F.Cu") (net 2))
 (segment (start 98.601 110.02605) (end 97.95605 110.671) (width 0.2) (layer "F.Cu") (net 2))
 (segment (start 136.585075 110.382) (end 136.252875 110.382) (width 0.2) (layer "F.Cu") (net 2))
 (segment (start 96.399 109.11395) (end 96.399 98.95605) (width 0.2) (layer "F.Cu") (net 2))
 (segment (start 150.107807 90.88) (end 131 90.88) (width 0.2) (layer "F.Cu") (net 2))
 (segment (start 98.62505 107.8) (end 97.95605 108.469) (width 0.2) (layer "F.Cu") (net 2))
 (segment (start 111.04 90.88) (end 112.041 89.879) (width 0.2) (layer "F.Cu") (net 2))
 (segment (start 97.95605 110.671) (end 97.04395 110.671) (width 0.2) (layer "F.Cu") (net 2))
 (segment (start 136.819975 110.1471) (end 136.585075 110.382) (width 0.2) (layer "F.Cu") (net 2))
 (segment (start 96.399 98.04395) (end 97.04395 97.399) (width 0.2) (layer "F.Cu") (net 2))
 (segment (start 148.007125 110.62) (end 144.104725 106.7176) (width 0.2) (layer "F.Cu") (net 2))
 (segment (start 124.0879 107.8) (end 123.67205 107.8) (width 0.2) (layer "F.Cu") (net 2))
 (segment (start 140.249475 106.7176) (end 139.167075 107.8) (width 0.2) (layer "F.Cu") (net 2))
 (segment (start 150.5 95.38) (end 150.5 91.272193) (width 0.2) (layer "F.Cu") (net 2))
 (segment (start 109.739 92.181) (end 111.04 90.88) (width 0.2) (layer "F.Cu") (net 2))
 (segment (start 136.418975 109.981) (end 141.899975 104.5) (width 0.2) (layer "F.Cu") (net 15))
 (segment (start 149.46 104.5) (end 150.5 105.54) (width 0.2) (layer "F.Cu") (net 15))
 (segment (start 141.899975 104.5) (end 149.46 104.5) (width 0.2) (layer "F.Cu") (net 15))
 (segment (start 126.836 109.981) (end 136.418975 109.981) (width 0.2) (layer "F.Cu") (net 15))
 (segment (start 123.195 106.34) (end 126.836 109.981) (width 0.2) (layer "F.Cu") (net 15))
 (segment (start 152.1218 105.141775) (end 152.1218 106.4582) (width 0.2) (layer "F.Cu") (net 14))
 (segment (start 151.079025 104.099) (end 152.1218 105.141775) (width 0.2) (layer "F.Cu") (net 14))
 (segment (start 133.056 104.099) (end 151.079025 104.099) (width 0.2) (layer "F.Cu") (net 14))
 (segment (start 130.815 106.34) (end 133.056 104.099) (width 0.2) (layer "F.Cu") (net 14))
 (segment (start 152.1218 106.4582) (end 150.5 108.08) (width 0.2) (layer "F.Cu") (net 14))
 (segment (start 130.69695 104.901) (end 131.599 104.901) (width 0.2) (layer "F.Cu") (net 16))
 (segment (start 129.714 105.88395) (end 130.69695 104.901) (width 0.2) (layer "F.Cu") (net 16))
 (segment (start 131.599 104.901) (end 135.0786 101.4214) (width 0.2) (layer "F.Cu") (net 16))
 (segment (start 135.0786 101.4214) (end 149.5386 101.4214) (width 0.2) (layer "F.Cu") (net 16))
 (segment (start 130.815 108.88) (end 129.714 107.779) (width 0.2) (layer "F.Cu") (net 16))
 (segment (start 149.5386 101.4214) (end 150.5 100.46) (width 0.2) (layer "F.Cu") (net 16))
 (segment (start 129.714 107.779) (end 129.714 105.88395) (width 0.2) (layer "F.Cu") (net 16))
 (segment (start 95.998 110.19215) (end 95.998 110.002) (width 0.2) (layer "F.Cu") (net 4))
 (segment (start 97.78995 96.998) (end 98.12215 96.998) (width 0.2) (layer "F.Cu") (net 4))
 (segment (start 141.2582 107.681775) (end 141.2582 111.5382) (width 0.2) (layer "F.Cu") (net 4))
 (segment (start 208.1665 104.1585) (end 208.1665 106.02426) (width 0.2) (layer "F.Cu") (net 4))
 (segment (start 96.64295 110.8371) (end 96.2329 110.42705) (width 0.2) (layer "F.Cu") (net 4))
 (segment (start 141.2582 111.5382) (end 142.88 113.16) (width 0.2) (layer "F.Cu") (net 4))
 (segment (start 177.481 122.981) (end 177.42395 122.981) (width 0.2) (layer "F.Cu") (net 4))
 (segment (start 143.938625 107.1186) (end 141.821375 107.1186) (width 0.2) (layer "F.Cu") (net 4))
 (segment (start 123.195 108.88) (end 121.003 111.072) (width 0.2) (layer "F.Cu") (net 4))
 (segment (start 163.981 129.981) (end 147.16 113.16) (width 0.2) (layer "F.Cu") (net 4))
 (segment (start 209.3175 103.0075) (end 208.1665 104.1585) (width 0.2) (layer "F.Cu") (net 4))
 (segment (start 178.33605 120.779) (end 178.981 121.42395) (width 0.2) (layer "F.Cu") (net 4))
 (segment (start 97.21005 111.072) (end 96.87785 111.072) (width 0.2) (layer "F.Cu") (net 4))
 (segment (start 96.64295 97.2329) (end 96.87785 96.998) (width 0.2) (layer "F.Cu") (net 4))
 (segment (start 218.0885 104.1585) (end 216.9375 103.0075) (width 0.2) (layer "F.Cu") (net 4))
 (segment (start 217.41426 106.6985) (end 218.0885 106.02426) (width 0.2) (layer "F.Cu") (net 4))
 (segment (start 178.981 121.42395) (end 178.981 122.33605) (width 0.2) (layer "F.Cu") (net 4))
 (segment (start 177.42395 122.981) (end 176.779 122.33605) (width 0.2) (layer "F.Cu") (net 4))
 (segment (start 147.16 113.16) (end 142.88 113.16) (width 0.2) (layer "F.Cu") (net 4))
 (segment (start 178.981 122.33605) (end 178.33605 122.981) (width 0.2) (layer "F.Cu") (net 4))
 (segment (start 96.87785 96.998) (end 97.21005 96.998) (width 0.2) (layer "F.Cu") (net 4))
 (segment (start 95.998 99.12215) (end 95.998 98.78995) (width 0.2) (layer "F.Cu") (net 4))
 (segment (start 95.998 98.78995) (end 95.998 98.21005) (width 0.2) (layer "F.Cu") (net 4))
 (segment (start 208.84074 106.6985) (end 217.41426 106.6985) (width 0.2) (layer "F.Cu") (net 4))
 (segment (start 160.55705 103) (end 178.33605 120.779) (width 0.2) (layer "F.Cu") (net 4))
 (segment (start 178.33605 122.981) (end 177.481 122.981) (width 0.2) (layer "F.Cu") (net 4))
 (segment (start 208.1665 106.02426) (end 208.84074 106.6985) (width 0.2) (layer "F.Cu") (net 4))
 (segment (start 141.821375 107.1186) (end 141.2582 107.681775) (width 0.2) (layer "F.Cu") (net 4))
 (segment (start 95.998 109.85995) (end 95.998 109.28005) (width 0.2) (layer "F.Cu") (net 4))
 (segment (start 95.998 110.002) (end 95.998 109.85995) (width 0.2) (layer "F.Cu") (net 4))
 (segment (start 98.12215 111.072) (end 97.78995 111.072) (width 0.2) (layer "F.Cu") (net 4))
 (segment (start 107.199 96.998) (end 107.199 92.181) (width 0.2) (layer "F.Cu") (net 4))
 (segment (start 97.78995 111.072) (end 97.21005 111.072) (width 0.2) (layer "F.Cu") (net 4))
 (segment (start 196.67176 129.981) (end 163.981 129.981) (width 0.2) (layer "F.Cu") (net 4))
 (segment (start 218.0885 104.1585) (end 218.0885 108.56426) (width 0.2) (layer "F.Cu") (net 4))
 (segment (start 95.998 98.21005) (end 95.998 97.87785) (width 0.2) (layer "F.Cu") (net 4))
 (segment (start 96.2329 97.64295) (end 96.64295 97.2329) (width 0.2) (layer "F.Cu") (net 4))
 (segment (start 95.998 97.87785) (end 96.2329 97.64295) (width 0.2) (layer "F.Cu") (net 4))
 (segment (start 150.5 103) (end 160.55705 103) (width 0.2) (layer "F.Cu") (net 4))
 (segment (start 218.0885 106.02426) (end 218.0885 104.1585) (width 0.2) (layer "F.Cu") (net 4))
 (segment (start 176.779 122.279) (end 166.6986 112.1986) (width 0.2) (layer "F.Cu") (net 4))
 (segment (start 95.998 109.28005) (end 95.998 108.94785) (width 0.2) (layer "F.Cu") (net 4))
 (segment (start 176.779 122.33605) (end 176.779 122.279) (width 0.2) (layer "F.Cu") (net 4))
 (segment (start 96.87785 111.072) (end 96.64295 110.8371) (width 0.2) (layer "F.Cu") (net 4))
 (segment (start 149.018625 112.1986) (end 143.938625 107.1186) (width 0.2) (layer "F.Cu") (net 4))
 (segment (start 98.12215 96.998) (end 107.199 96.998) (width 0.2) (layer "F.Cu") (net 4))
 (segment (start 121.003 111.072) (end 98.12215 111.072) (width 0.2) (layer "F.Cu") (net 4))
 (segment (start 218.0885 108.56426) (end 196.67176 129.981) (width 0.2) (layer "F.Cu") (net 4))
 (segment (start 95.998 108.94785) (end 95.998 99.12215) (width 0.2) (layer "F.Cu") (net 4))
 (segment (start 127.475 113.16) (end 142.88 113.16) (width 0.2) (layer "F.Cu") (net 4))
 (segment (start 96.2329 110.42705) (end 95.998 110.19215) (width 0.2) (layer "F.Cu") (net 4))
 (segment (start 166.6986 112.1986) (end 149.018625 112.1986) (width 0.2) (layer "F.Cu") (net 4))
 (segment (start 107.199 92.181) (end 108.5 90.88) (width 0.2) (layer "F.Cu") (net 4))
 (segment (start 123.195 108.88) (end 127.475 113.16) (width 0.2) (layer "F.Cu") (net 4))
 (segment (start 97.21005 96.998) (end 97.78995 96.998) (width 0.2) (layer "F.Cu") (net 4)))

